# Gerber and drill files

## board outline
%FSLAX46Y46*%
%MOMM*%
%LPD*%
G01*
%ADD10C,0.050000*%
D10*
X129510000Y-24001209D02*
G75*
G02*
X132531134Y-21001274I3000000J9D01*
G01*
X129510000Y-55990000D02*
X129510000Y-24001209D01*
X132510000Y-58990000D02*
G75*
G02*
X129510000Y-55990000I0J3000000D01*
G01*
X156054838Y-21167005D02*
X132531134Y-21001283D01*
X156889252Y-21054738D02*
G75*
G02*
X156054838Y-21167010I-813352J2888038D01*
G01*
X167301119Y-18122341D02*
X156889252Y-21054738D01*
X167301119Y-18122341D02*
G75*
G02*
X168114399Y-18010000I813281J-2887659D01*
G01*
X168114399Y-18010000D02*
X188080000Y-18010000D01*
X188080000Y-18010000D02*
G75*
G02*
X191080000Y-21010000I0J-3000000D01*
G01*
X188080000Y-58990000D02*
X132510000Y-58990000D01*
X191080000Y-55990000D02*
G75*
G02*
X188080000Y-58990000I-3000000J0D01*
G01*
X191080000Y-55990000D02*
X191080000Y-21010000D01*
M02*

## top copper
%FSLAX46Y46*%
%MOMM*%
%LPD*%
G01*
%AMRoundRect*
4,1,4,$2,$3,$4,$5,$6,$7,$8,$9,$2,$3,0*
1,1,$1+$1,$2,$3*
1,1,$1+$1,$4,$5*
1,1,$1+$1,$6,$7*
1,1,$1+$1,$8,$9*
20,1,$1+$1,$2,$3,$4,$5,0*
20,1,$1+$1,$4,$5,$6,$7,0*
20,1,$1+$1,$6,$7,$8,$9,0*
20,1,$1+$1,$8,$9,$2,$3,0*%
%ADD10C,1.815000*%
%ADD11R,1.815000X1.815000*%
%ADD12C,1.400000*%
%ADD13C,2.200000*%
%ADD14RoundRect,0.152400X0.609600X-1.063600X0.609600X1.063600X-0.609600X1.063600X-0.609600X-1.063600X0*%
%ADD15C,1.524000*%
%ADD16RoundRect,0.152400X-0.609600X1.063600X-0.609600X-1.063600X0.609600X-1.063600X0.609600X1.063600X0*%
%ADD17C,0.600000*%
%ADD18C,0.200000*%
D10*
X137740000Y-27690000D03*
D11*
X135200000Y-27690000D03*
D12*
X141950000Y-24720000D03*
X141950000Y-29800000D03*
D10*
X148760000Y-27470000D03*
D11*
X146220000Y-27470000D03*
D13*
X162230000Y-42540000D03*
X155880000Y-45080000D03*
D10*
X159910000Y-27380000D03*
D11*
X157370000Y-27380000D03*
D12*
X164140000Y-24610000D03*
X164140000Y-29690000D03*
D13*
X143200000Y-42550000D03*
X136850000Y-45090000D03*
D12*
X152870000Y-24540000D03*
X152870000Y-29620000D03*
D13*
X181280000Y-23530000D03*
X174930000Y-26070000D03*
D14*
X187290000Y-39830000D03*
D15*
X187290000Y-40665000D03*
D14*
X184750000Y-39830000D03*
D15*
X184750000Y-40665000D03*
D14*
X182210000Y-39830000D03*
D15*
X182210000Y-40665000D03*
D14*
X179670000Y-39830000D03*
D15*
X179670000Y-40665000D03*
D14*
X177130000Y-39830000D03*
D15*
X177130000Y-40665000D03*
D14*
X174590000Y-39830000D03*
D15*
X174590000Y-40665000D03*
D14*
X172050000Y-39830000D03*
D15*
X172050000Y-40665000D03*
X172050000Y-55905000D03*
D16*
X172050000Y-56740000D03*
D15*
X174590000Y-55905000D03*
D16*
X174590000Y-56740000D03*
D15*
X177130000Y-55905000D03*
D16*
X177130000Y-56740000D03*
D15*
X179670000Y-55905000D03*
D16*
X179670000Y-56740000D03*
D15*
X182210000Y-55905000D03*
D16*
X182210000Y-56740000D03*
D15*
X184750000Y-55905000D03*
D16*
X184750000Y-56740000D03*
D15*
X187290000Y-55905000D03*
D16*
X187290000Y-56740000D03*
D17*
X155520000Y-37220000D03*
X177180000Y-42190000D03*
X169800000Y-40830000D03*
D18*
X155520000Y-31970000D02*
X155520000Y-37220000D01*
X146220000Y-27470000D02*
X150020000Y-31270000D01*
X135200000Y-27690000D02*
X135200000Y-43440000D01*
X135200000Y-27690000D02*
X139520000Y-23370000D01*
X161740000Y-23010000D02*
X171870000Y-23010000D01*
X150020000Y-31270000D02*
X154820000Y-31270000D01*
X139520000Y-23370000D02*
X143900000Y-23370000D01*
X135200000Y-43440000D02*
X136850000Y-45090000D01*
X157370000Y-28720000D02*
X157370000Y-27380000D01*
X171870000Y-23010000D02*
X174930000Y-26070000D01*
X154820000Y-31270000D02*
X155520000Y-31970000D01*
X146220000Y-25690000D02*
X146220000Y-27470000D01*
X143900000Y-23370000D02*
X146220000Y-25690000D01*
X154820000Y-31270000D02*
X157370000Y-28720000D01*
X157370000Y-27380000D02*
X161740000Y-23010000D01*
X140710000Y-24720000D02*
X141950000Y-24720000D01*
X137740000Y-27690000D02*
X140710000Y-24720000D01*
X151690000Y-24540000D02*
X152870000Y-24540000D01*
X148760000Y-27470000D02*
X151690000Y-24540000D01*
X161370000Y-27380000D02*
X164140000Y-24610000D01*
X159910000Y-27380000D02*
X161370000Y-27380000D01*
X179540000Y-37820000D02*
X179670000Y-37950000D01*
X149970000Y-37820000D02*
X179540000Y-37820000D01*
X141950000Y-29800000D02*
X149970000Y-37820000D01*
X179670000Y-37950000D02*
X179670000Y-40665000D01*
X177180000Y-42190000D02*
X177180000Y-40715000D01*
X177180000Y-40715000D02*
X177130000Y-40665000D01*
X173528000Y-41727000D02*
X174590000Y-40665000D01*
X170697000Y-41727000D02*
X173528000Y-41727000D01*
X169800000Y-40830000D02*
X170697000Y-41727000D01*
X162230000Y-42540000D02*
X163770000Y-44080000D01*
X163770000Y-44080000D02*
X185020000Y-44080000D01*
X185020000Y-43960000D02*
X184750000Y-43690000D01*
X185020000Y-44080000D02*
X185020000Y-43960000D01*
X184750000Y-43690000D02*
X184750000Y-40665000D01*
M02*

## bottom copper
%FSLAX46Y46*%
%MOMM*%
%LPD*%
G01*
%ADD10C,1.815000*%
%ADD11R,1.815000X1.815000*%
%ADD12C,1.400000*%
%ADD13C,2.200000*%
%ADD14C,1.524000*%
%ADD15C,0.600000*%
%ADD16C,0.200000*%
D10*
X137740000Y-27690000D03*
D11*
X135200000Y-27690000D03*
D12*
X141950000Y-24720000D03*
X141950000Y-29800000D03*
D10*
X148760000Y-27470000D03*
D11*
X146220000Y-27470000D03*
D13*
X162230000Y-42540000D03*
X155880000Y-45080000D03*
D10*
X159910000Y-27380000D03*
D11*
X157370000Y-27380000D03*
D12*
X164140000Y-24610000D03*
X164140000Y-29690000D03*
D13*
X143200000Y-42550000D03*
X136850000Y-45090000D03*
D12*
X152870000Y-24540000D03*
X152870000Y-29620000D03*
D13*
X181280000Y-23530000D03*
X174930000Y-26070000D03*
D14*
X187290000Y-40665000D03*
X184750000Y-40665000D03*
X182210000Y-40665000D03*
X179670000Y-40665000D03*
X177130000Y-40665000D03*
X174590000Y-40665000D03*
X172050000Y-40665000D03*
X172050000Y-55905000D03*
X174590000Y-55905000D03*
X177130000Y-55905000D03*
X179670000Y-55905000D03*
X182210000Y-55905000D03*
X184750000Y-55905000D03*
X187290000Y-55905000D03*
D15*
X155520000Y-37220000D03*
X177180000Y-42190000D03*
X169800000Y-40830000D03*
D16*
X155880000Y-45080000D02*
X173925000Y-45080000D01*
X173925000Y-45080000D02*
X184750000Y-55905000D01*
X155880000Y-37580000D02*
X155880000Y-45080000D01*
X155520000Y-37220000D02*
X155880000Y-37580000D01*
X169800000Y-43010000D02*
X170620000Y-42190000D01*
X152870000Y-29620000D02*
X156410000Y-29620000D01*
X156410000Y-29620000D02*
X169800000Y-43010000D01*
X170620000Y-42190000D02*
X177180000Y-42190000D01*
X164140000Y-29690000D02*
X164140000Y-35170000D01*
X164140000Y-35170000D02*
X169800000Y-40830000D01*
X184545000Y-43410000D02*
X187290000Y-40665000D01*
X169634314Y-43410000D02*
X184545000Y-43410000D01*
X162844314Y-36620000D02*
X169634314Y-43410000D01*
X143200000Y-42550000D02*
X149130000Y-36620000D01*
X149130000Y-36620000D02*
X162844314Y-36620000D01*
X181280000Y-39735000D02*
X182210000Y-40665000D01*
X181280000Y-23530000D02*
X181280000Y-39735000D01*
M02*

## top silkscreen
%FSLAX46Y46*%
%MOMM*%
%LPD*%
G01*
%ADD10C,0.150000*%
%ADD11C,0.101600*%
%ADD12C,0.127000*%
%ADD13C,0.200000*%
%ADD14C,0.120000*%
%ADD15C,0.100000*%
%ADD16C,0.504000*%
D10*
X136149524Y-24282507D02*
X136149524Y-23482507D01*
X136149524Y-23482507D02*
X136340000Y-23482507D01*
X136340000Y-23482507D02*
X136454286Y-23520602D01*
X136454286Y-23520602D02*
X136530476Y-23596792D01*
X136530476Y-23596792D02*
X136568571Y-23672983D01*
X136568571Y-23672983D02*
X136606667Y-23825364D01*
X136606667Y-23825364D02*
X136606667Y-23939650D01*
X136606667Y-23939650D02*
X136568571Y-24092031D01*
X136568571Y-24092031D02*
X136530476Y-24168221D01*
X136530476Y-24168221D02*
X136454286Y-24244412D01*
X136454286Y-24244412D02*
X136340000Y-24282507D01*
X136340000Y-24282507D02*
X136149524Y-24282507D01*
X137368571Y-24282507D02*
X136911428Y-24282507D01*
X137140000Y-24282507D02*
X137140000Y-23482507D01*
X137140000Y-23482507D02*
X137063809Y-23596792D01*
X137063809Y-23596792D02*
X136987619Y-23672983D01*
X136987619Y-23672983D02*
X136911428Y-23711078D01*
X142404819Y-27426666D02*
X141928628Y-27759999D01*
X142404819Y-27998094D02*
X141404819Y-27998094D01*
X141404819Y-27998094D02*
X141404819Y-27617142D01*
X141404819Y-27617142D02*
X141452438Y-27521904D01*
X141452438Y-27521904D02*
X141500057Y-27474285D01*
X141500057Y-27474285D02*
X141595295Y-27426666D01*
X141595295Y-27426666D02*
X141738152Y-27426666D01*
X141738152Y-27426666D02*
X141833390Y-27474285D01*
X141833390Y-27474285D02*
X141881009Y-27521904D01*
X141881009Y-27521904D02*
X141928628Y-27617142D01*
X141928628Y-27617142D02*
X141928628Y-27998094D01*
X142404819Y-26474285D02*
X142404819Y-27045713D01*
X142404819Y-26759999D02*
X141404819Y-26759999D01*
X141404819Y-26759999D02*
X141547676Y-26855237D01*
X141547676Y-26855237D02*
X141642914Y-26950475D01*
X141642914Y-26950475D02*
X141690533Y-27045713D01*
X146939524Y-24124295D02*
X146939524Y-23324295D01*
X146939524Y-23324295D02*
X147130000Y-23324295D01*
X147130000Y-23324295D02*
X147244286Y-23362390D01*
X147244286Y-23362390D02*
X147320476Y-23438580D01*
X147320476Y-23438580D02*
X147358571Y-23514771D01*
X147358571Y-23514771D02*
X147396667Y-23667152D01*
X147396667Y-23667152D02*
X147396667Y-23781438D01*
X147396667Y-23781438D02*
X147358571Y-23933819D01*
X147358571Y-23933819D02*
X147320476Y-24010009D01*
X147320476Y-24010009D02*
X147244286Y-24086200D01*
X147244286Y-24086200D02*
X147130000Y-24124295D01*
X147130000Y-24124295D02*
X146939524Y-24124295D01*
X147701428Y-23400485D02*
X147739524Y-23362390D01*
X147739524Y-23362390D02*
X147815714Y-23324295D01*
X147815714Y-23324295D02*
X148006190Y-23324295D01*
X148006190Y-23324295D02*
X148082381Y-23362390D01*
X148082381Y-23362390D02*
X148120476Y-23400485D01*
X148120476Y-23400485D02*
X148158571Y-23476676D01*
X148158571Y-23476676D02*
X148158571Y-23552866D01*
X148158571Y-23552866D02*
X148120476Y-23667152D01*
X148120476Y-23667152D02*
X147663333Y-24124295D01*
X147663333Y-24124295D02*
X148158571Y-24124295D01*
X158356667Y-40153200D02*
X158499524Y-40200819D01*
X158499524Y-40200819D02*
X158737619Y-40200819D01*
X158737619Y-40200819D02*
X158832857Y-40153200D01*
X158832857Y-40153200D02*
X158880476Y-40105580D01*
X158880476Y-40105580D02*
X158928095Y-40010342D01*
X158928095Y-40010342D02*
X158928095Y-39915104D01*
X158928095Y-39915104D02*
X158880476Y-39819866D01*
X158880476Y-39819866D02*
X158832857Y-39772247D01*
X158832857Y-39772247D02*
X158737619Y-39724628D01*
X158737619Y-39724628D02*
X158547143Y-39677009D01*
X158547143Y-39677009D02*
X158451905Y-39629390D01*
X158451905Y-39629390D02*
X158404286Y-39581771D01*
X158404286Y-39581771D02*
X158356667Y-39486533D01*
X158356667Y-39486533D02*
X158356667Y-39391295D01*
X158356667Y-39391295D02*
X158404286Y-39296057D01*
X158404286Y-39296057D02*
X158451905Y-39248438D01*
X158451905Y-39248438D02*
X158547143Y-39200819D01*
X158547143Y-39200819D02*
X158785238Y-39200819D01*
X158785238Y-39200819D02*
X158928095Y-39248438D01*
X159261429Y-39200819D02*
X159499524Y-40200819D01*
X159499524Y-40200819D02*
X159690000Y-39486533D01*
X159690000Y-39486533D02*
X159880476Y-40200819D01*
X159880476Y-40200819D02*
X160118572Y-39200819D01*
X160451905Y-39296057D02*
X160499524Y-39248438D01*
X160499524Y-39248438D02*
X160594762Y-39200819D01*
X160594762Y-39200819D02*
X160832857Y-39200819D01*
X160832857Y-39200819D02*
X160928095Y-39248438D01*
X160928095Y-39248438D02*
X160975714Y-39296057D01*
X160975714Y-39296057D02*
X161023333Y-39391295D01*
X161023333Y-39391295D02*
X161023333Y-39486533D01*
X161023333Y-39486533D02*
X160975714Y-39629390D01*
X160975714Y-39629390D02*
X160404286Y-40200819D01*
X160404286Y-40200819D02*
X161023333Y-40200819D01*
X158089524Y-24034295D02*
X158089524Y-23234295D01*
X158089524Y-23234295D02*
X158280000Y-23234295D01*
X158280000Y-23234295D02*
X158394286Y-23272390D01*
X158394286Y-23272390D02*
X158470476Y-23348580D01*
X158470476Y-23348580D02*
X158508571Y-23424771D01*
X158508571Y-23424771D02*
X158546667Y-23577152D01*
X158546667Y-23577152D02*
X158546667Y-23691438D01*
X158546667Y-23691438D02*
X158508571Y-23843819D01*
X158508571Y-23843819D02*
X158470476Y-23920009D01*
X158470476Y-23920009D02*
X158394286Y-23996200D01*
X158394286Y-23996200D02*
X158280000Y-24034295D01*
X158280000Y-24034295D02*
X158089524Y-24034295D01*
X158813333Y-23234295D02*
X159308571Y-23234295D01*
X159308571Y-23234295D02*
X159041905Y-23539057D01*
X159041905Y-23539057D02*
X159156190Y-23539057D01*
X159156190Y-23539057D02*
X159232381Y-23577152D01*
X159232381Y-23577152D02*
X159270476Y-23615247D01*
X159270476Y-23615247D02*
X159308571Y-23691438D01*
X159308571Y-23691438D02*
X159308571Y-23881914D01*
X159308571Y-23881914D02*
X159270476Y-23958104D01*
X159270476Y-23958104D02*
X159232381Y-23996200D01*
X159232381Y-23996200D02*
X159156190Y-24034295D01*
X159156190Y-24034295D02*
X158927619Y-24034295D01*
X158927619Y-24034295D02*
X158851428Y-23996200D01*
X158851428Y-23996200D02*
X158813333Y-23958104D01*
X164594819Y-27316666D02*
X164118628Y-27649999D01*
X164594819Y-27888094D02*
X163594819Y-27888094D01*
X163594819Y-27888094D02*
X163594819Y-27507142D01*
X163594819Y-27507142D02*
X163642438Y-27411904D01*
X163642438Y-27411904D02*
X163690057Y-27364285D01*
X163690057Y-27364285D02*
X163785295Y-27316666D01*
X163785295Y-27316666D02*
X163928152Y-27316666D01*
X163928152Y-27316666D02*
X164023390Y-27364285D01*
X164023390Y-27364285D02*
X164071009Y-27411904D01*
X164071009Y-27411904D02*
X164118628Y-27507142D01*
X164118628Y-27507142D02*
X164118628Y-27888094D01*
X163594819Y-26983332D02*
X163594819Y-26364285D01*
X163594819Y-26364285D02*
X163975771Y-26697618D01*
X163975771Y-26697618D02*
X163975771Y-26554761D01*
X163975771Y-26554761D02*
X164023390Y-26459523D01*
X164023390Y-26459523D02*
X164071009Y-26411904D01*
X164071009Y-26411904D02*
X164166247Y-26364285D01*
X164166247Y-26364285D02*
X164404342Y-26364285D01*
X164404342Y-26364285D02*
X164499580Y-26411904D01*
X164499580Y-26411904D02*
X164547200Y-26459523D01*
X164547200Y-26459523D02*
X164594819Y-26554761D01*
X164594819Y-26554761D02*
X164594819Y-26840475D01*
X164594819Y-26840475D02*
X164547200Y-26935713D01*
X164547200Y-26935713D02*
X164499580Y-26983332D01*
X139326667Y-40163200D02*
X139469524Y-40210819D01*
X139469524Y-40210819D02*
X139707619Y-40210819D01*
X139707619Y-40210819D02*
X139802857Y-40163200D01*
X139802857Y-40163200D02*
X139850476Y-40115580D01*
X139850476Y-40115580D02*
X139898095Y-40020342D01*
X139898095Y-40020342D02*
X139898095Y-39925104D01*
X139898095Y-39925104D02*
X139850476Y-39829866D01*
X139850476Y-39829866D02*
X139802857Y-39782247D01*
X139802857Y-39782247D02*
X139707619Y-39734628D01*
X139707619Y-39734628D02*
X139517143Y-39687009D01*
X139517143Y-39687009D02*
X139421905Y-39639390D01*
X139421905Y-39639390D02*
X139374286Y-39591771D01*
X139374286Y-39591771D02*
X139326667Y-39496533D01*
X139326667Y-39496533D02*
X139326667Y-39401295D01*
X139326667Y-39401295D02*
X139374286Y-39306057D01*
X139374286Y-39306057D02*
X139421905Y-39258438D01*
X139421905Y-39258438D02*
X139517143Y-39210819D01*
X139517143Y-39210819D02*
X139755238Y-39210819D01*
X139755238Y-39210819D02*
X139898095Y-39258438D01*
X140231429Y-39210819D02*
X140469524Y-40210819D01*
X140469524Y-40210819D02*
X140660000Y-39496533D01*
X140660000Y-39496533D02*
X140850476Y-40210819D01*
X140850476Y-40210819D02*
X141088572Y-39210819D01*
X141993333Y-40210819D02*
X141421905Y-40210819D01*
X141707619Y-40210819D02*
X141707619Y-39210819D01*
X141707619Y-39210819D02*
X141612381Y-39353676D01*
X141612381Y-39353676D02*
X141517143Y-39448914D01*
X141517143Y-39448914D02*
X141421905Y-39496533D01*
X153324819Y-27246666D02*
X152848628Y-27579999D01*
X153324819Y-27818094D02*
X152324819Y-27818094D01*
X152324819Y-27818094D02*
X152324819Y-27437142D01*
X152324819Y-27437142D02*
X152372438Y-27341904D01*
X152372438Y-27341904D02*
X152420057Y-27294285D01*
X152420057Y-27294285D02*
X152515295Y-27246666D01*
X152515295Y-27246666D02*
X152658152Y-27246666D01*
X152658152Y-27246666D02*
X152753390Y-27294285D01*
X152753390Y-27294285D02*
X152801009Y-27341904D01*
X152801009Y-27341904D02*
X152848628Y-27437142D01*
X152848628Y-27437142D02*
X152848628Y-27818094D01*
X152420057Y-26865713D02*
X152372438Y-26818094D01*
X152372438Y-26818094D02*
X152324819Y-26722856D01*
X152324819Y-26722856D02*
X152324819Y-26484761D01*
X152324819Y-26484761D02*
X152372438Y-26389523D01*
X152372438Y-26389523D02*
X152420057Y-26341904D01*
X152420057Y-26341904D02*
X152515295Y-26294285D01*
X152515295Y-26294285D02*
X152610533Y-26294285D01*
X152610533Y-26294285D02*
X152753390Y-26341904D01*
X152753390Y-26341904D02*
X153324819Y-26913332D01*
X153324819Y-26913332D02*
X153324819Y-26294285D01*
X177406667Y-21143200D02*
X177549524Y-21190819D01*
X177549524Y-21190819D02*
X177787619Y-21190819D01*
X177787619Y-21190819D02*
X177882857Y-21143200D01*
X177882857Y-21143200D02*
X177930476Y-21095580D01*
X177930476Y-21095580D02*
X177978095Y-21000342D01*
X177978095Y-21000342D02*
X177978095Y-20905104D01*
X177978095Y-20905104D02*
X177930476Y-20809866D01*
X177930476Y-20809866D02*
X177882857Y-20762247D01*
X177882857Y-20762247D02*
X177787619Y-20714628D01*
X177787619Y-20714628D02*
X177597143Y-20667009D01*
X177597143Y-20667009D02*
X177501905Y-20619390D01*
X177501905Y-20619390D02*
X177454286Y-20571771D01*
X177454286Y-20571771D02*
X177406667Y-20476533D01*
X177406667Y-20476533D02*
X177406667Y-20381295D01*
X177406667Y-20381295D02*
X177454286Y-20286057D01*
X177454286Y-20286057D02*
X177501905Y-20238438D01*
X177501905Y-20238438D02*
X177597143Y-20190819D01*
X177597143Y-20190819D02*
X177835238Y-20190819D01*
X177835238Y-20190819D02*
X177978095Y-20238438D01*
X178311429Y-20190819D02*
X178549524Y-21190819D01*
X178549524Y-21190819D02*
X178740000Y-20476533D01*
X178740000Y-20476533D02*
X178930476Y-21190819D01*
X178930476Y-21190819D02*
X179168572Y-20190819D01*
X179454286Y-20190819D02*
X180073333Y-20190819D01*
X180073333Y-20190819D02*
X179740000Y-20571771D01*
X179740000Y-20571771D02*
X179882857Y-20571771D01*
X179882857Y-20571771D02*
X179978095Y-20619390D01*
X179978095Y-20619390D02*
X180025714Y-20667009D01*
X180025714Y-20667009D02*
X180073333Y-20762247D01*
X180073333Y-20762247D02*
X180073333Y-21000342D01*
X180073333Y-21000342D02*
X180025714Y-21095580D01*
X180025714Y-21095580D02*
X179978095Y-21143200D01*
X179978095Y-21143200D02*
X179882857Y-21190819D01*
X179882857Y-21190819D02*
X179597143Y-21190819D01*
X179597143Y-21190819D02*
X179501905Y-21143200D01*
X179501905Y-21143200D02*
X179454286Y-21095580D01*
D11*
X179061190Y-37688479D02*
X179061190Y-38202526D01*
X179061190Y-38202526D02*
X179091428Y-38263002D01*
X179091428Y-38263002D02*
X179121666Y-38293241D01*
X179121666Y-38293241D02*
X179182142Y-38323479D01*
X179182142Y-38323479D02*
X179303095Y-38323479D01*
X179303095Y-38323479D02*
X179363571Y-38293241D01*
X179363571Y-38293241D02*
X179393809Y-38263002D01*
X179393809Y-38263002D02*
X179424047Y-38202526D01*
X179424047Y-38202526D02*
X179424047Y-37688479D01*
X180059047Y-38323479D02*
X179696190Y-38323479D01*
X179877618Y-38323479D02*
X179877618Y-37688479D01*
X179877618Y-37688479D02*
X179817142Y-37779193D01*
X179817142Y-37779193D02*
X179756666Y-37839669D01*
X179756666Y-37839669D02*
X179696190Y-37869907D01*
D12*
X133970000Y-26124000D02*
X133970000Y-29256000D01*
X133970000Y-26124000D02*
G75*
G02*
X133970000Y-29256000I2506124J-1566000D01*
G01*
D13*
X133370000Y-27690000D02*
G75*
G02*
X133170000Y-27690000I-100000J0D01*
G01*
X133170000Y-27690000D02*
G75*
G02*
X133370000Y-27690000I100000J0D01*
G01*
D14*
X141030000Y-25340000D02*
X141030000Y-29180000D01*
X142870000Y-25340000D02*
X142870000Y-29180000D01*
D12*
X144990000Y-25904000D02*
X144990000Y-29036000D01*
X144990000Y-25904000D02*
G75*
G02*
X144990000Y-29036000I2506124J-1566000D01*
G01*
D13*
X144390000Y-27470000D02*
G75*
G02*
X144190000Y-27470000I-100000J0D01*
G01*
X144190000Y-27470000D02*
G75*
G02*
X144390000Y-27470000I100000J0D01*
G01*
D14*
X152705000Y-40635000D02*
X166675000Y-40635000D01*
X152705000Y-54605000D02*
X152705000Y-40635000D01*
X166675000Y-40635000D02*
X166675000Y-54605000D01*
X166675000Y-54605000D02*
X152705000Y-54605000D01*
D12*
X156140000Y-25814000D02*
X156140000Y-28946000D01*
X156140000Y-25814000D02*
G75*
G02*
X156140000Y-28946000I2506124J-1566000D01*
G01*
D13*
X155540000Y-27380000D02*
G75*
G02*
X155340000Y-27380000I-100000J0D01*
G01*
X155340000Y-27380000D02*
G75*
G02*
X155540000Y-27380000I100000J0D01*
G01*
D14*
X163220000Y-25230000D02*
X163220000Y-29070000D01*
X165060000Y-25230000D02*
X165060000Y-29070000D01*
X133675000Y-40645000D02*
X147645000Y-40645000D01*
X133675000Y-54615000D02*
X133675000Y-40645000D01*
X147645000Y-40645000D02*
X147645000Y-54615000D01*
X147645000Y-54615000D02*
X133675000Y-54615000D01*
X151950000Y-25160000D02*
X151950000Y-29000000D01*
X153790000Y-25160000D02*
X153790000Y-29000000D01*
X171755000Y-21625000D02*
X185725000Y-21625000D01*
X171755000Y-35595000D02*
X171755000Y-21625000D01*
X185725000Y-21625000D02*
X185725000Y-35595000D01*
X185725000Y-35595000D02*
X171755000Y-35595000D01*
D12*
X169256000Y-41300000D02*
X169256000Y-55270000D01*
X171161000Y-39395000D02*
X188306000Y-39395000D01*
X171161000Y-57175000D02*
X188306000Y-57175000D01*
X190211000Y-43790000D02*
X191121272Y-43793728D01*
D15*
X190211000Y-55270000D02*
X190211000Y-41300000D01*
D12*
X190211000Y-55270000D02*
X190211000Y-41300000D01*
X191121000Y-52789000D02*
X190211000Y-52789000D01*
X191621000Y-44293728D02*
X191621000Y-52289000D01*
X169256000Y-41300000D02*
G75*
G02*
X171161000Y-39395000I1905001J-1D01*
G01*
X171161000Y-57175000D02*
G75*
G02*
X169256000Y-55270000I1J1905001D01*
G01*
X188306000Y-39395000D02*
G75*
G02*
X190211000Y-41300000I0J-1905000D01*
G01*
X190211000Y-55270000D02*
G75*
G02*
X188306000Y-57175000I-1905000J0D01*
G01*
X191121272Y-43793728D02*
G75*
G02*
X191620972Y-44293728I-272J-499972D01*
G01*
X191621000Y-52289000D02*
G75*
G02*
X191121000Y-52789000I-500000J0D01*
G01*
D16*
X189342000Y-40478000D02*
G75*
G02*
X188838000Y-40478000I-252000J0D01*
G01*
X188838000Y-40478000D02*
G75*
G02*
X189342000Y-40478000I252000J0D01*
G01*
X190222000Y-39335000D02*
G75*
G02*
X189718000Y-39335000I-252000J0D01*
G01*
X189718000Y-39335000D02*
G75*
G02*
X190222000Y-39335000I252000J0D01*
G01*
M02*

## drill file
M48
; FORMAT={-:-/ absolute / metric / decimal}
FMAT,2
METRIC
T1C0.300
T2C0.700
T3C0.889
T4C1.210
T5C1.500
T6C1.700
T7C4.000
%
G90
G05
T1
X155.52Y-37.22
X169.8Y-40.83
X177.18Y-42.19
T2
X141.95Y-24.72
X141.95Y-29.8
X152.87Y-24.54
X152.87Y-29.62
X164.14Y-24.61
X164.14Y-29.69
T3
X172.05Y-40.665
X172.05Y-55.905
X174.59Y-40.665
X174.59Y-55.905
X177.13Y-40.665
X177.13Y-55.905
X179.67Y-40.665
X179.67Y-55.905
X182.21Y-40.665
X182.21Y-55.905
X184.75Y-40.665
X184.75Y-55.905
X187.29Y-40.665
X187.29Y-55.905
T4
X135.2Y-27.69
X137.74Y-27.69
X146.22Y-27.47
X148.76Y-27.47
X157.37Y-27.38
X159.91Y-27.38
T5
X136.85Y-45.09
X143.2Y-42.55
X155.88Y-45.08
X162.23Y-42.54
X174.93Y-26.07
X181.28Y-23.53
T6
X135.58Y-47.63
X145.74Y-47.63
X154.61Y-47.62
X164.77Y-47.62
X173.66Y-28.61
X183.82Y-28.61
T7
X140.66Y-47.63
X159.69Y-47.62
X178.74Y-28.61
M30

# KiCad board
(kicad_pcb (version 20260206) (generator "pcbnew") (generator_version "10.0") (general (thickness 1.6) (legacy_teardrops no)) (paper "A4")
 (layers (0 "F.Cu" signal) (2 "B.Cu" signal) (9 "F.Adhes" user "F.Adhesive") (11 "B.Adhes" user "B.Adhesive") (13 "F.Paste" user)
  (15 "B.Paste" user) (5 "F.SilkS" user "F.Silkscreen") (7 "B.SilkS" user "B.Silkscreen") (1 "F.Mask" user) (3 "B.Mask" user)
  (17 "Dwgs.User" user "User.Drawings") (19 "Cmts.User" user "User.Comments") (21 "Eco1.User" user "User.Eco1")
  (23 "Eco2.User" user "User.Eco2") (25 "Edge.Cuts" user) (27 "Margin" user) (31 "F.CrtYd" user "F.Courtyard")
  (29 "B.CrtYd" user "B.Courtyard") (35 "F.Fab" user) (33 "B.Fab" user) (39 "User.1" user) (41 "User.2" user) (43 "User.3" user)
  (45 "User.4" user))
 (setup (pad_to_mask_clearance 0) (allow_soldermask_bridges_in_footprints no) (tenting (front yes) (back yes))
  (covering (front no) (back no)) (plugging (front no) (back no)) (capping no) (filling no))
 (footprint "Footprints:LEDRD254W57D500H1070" (layer "F.Cu") (at 136.47 27.69)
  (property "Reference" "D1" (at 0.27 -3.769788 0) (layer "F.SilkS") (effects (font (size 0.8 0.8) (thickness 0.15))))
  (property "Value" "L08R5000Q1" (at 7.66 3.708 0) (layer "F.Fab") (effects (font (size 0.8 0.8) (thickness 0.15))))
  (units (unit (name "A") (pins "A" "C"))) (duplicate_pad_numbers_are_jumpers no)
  (fp_line (start -2.5 -1.566) (end -2.5 1.566) (stroke (width 0.127) (type solid)) (layer "F.SilkS"))
  (fp_arc (start -2.5 -1.566) (mid 2.961291 0) (end -2.5 1.566) (stroke (width 0.127) (type solid)) (layer "F.SilkS"))
  (fp_circle (center -3.2 0) (end -3.1 0) (stroke (width 0.2) (type solid)) (fill no) (layer "F.SilkS"))
  (pad "A" thru_hole circle (at 1.27 0) (size 1.815 1.815) (drill 1.21) (layers "*.Cu" "*.Mask") (remove_unused_layers no)
   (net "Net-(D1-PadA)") (solder_mask_margin 0.102))
  (pad "C" thru_hole rect (at -1.27 0) (size 1.815 1.815) (drill 1.21) (layers "*.Cu" "*.Mask") (remove_unused_layers no) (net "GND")
   (solder_mask_margin 0.102)))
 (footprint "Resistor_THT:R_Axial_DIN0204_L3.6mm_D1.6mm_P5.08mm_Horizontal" (layer "F.Cu") (at 141.95 24.72 -90)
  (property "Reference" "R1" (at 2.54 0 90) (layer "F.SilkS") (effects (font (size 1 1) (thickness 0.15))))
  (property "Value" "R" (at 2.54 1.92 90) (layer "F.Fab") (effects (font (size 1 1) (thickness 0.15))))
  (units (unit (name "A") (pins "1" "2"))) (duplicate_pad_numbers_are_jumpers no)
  (fp_line (start 0.62 0.92) (end 4.46 0.92) (stroke (width 0.12) (type solid)) (layer "F.SilkS"))
  (fp_line (start 0.62 -0.92) (end 4.46 -0.92) (stroke (width 0.12) (type solid)) (layer "F.SilkS"))
  (pad "1" thru_hole circle (at 0 0 270) (size 1.4 1.4) (drill 0.7) (layers "*.Cu" "*.Mask") (remove_unused_layers no) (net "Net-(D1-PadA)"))
  (pad "2" thru_hole circle (at 5.08 0 270) (size 1.4 1.4) (drill 0.7) (layers "*.Cu" "*.Mask") (remove_unused_layers no) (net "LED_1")))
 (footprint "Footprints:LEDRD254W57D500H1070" (layer "F.Cu") (at 147.49 27.47)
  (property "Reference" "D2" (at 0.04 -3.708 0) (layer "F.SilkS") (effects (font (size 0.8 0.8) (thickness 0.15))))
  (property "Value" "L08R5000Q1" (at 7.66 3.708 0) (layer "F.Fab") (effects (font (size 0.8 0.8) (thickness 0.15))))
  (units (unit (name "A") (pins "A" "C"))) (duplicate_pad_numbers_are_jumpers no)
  (fp_line (start -2.5 -1.566) (end -2.5 1.566) (stroke (width 0.127) (type solid)) (layer "F.SilkS"))
  (fp_arc (start -2.5 -1.566) (mid 2.961291 0) (end -2.5 1.566) (stroke (width 0.127) (type solid)) (layer "F.SilkS"))
  (fp_circle (center -3.2 0) (end -3.1 0) (stroke (width 0.2) (type solid)) (fill no) (layer "F.SilkS"))
  (pad "A" thru_hole circle (at 1.27 0) (size 1.815 1.815) (drill 1.21) (layers "*.Cu" "*.Mask") (remove_unused_layers no)
   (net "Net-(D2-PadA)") (solder_mask_margin 0.102))
  (pad "C" thru_hole rect (at -1.27 0) (size 1.815 1.815) (drill 1.21) (layers "*.Cu" "*.Mask") (remove_unused_layers no) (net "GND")
   (solder_mask_margin 0.102)))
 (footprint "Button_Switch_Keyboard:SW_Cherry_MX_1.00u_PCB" (layer "F.Cu") (at 162.23 42.54)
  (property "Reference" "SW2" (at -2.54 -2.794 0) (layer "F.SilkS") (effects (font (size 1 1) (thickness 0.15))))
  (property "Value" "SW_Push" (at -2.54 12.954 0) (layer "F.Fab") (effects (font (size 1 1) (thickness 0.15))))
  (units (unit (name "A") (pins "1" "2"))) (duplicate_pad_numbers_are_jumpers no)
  (fp_line (start -9.525 -1.905) (end 4.445 -1.905) (stroke (width 0.12) (type solid)) (layer "F.SilkS"))
  (fp_line (start -9.525 12.065) (end -9.525 -1.905) (stroke (width 0.12) (type solid)) (layer "F.SilkS"))
  (fp_line (start 4.445 -1.905) (end 4.445 12.065) (stroke (width 0.12) (type solid)) (layer "F.SilkS"))
  (fp_line (start 4.445 12.065) (end -9.525 12.065) (stroke (width 0.12) (type solid)) (layer "F.SilkS"))
  (pad "" np_thru_hole circle (at -7.62 5.08) (size 1.7 1.7) (drill 1.7) (layers "*.Cu" "*.Mask"))
  (pad "" np_thru_hole circle (at -2.54 5.08) (size 4 4) (drill 4) (layers "*.Cu" "*.Mask"))
  (pad "" np_thru_hole circle (at 2.54 5.08) (size 1.7 1.7) (drill 1.7) (layers "*.Cu" "*.Mask"))
  (pad "1" thru_hole circle (at 0 0) (size 2.2 2.2) (drill 1.5) (layers "*.Cu" "*.Mask") (remove_unused_layers no) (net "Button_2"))
  (pad "2" thru_hole circle (at -6.35 2.54) (size 2.2 2.2) (drill 1.5) (layers "*.Cu" "*.Mask") (remove_unused_layers no) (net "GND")))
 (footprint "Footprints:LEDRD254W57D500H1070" (layer "F.Cu") (at 158.64 27.38)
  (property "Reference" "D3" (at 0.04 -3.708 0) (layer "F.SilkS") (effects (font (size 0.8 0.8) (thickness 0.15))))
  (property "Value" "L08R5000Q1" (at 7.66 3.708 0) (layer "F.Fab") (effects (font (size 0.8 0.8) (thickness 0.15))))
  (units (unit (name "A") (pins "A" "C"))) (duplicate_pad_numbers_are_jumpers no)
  (fp_line (start -2.5 -1.566) (end -2.5 1.566) (stroke (width 0.127) (type solid)) (layer "F.SilkS"))
  (fp_arc (start -2.5 -1.566) (mid 2.961291 0) (end -2.5 1.566) (stroke (width 0.127) (type solid)) (layer "F.SilkS"))
  (fp_circle (center -3.2 0) (end -3.1 0) (stroke (width 0.2) (type solid)) (fill no) (layer "F.SilkS"))
  (pad "A" thru_hole circle (at 1.27 0) (size 1.815 1.815) (drill 1.21) (layers "*.Cu" "*.Mask") (remove_unused_layers no)
   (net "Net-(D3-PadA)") (solder_mask_margin 0.102))
  (pad "C" thru_hole rect (at -1.27 0) (size 1.815 1.815) (drill 1.21) (layers "*.Cu" "*.Mask") (remove_unused_layers no) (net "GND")
   (solder_mask_margin 0.102)))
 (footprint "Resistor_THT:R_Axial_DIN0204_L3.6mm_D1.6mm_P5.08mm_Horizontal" (layer "F.Cu") (at 164.14 24.61 -90)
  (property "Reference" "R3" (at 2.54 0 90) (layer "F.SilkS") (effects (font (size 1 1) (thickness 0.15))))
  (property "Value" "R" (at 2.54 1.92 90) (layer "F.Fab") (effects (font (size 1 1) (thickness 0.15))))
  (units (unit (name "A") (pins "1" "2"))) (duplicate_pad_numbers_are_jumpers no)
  (fp_line (start 0.62 0.92) (end 4.46 0.92) (stroke (width 0.12) (type solid)) (layer "F.SilkS"))
  (fp_line (start 0.62 -0.92) (end 4.46 -0.92) (stroke (width 0.12) (type solid)) (layer "F.SilkS"))
  (pad "1" thru_hole circle (at 0 0 270) (size 1.4 1.4) (drill 0.7) (layers "*.Cu" "*.Mask") (remove_unused_layers no) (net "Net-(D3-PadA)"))
  (pad "2" thru_hole circle (at 5.08 0 270) (size 1.4 1.4) (drill 0.7) (layers "*.Cu" "*.Mask") (remove_unused_layers no) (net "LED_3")))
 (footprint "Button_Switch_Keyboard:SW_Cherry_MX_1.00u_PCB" (layer "F.Cu") (at 143.2 42.55)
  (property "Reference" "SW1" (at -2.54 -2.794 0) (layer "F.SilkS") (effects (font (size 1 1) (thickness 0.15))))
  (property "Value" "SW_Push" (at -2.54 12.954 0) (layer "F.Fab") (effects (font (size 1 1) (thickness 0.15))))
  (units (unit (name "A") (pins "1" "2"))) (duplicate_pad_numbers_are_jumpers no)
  (fp_line (start -9.525 -1.905) (end 4.445 -1.905) (stroke (width 0.12) (type solid)) (layer "F.SilkS"))
  (fp_line (start -9.525 12.065) (end -9.525 -1.905) (stroke (width 0.12) (type solid)) (layer "F.SilkS"))
  (fp_line (start 4.445 -1.905) (end 4.445 12.065) (stroke (width 0.12) (type solid)) (layer "F.SilkS"))
  (fp_line (start 4.445 12.065) (end -9.525 12.065) (stroke (width 0.12) (type solid)) (layer "F.SilkS"))
  (pad "" np_thru_hole circle (at -7.62 5.08) (size 1.7 1.7) (drill 1.7) (layers "*.Cu" "*.Mask"))
  (pad "" np_thru_hole circle (at -2.54 5.08) (size 4 4) (drill 4) (layers "*.Cu" "*.Mask"))
  (pad "" np_thru_hole circle (at 2.54 5.08) (size 1.7 1.7) (drill 1.7) (layers "*.Cu" "*.Mask"))
  (pad "1" thru_hole circle (at 0 0) (size 2.2 2.2) (drill 1.5) (layers "*.Cu" "*.Mask") (remove_unused_layers no) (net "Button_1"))
  (pad "2" thru_hole circle (at -6.35 2.54) (size 2.2 2.2) (drill 1.5) (layers "*.Cu" "*.Mask") (remove_unused_layers no) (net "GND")))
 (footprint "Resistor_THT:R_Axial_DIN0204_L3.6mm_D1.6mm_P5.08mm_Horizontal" (layer "F.Cu") (at 152.87 24.54 -90)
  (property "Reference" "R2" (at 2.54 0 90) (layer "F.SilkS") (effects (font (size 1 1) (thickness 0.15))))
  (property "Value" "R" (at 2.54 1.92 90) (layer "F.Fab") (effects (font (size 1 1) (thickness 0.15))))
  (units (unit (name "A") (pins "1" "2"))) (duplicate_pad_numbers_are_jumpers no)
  (fp_line (start 0.62 0.92) (end 4.46 0.92) (stroke (width 0.12) (type solid)) (layer "F.SilkS"))
  (fp_line (start 0.62 -0.92) (end 4.46 -0.92) (stroke (width 0.12) (type solid)) (layer "F.SilkS"))
  (pad "1" thru_hole circle (at 0 0 270) (size 1.4 1.4) (drill 0.7) (layers "*.Cu" "*.Mask") (remove_unused_layers no) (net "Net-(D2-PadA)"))
  (pad "2" thru_hole circle (at 5.08 0 270) (size 1.4 1.4) (drill 0.7) (layers "*.Cu" "*.Mask") (remove_unused_layers no) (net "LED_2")))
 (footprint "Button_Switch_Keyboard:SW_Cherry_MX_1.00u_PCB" (layer "F.Cu") (at 181.28 23.53)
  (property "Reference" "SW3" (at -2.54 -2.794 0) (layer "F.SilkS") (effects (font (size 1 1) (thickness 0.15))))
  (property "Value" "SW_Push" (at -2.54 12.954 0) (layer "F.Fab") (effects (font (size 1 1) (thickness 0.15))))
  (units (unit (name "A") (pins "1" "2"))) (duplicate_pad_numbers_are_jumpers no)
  (fp_line (start -9.525 -1.905) (end 4.445 -1.905) (stroke (width 0.12) (type solid)) (layer "F.SilkS"))
  (fp_line (start -9.525 12.065) (end -9.525 -1.905) (stroke (width 0.12) (type solid)) (layer "F.SilkS"))
  (fp_line (start 4.445 -1.905) (end 4.445 12.065) (stroke (width 0.12) (type solid)) (layer "F.SilkS"))
  (fp_line (start 4.445 12.065) (end -9.525 12.065) (stroke (width 0.12) (type solid)) (layer "F.SilkS"))
  (pad "" np_thru_hole circle (at -7.62 5.08) (size 1.7 1.7) (drill 1.7) (layers "*.Cu" "*.Mask"))
  (pad "" np_thru_hole circle (at -2.54 5.08) (size 4 4) (drill 4) (layers "*.Cu" "*.Mask"))
  (pad "" np_thru_hole circle (at 2.54 5.08) (size 1.7 1.7) (drill 1.7) (layers "*.Cu" "*.Mask"))
  (pad "1" thru_hole circle (at 0 0) (size 2.2 2.2) (drill 1.5) (layers "*.Cu" "*.Mask") (remove_unused_layers no) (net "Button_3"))
  (pad "2" thru_hole circle (at -6.35 2.54) (size 2.2 2.2) (drill 1.5) (layers "*.Cu" "*.Mask") (remove_unused_layers no) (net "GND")))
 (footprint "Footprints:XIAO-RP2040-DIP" (layer "F.Cu") (at 179.67 48.285)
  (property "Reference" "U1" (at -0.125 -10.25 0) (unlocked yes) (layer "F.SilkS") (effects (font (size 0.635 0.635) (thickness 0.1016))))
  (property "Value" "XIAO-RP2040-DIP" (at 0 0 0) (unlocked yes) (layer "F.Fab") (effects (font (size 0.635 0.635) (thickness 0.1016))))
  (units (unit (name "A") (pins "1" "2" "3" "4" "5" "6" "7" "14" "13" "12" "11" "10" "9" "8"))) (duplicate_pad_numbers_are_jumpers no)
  (fp_line (start -10.414 -6.985) (end -10.414 6.985) (stroke (width 0.127) (type solid)) (layer "F.SilkS"))
  (fp_line (start -8.509 -8.89) (end 8.636 -8.89) (stroke (width 0.127) (type solid)) (layer "F.SilkS"))
  (fp_line (start -8.509 8.89) (end 8.636 8.89) (stroke (width 0.127) (type solid)) (layer "F.SilkS"))
  (fp_line (start 10.541 -4.495) (end 11.451272 -4.491272) (stroke (width 0.127) (type solid)) (layer "F.SilkS"))
  (fp_line (start 10.541 6.985) (end 10.541 -6.985) (stroke (width 0.1) (type solid)) (layer "F.SilkS"))
  (fp_line (start 10.541 6.985) (end 10.541 -6.985) (stroke (width 0.127) (type solid)) (layer "F.SilkS"))
  (fp_line (start 11.451 4.504) (end 10.541 4.504) (stroke (width 0.127) (type solid)) (layer "F.SilkS"))
  (fp_line (start 11.951 -3.991272) (end 11.951 4.004) (stroke (width 0.127) (type solid)) (layer "F.SilkS"))
  (fp_arc (start -10.414 -6.985) (mid -9.856038 -8.332038) (end -8.509 -8.89) (stroke (width 0.127) (type solid)) (layer "F.SilkS"))
  (fp_arc (start -8.509 8.89) (mid -9.856038 8.332038) (end -10.414 6.985) (stroke (width 0.127) (type solid)) (layer "F.SilkS"))
  (fp_arc (start 8.636 -8.89) (mid 9.983038 -8.332038) (end 10.541 -6.985) (stroke (width 0.127) (type solid)) (layer "F.SilkS"))
  (fp_arc (start 10.541 6.985) (mid 9.983038 8.332038) (end 8.636 8.89) (stroke (width 0.127) (type solid)) (layer "F.SilkS"))
  (fp_arc (start 11.451272 -4.491272) (mid 11.804644 -4.344724) (end 11.951 -3.991272) (stroke (width 0.127) (type default))
   (layer "F.SilkS"))
  (fp_arc (start 11.951 4.004) (mid 11.804553 4.357553) (end 11.451 4.504) (stroke (width 0.127) (type default)) (layer "F.SilkS"))
  (fp_circle (center 9.42 -7.807) (end 9.674 -7.807) (stroke (width 0.5) (type solid)) (fill yes) (layer "F.SilkS"))
  (fp_circle (center 10.3 -8.95) (end 10.554 -8.95) (stroke (width 0.5) (type solid)) (fill yes) (layer "F.SilkS"))
  (pad "1" smd roundrect (at 7.62 -8.455 90) (size 2.432 1.524) (layers "F.Cu" "F.Mask") (roundrect_rratio 0.1) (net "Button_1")
   (thermal_bridge_angle 45))
  (pad "1" thru_hole circle (at 7.62 -7.62 90) (size 1.524 1.524) (drill 0.889) (layers "*.Cu" "*.Mask") (remove_unused_layers no)
   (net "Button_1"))
  (pad "2" smd roundrect (at 5.08 -8.455 90) (size 2.432 1.524) (layers "F.Cu" "F.Mask") (roundrect_rratio 0.1) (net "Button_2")
   (thermal_bridge_angle 45))
  (pad "2" thru_hole circle (at 5.08 -7.62 90) (size 1.524 1.524) (drill 0.889) (layers "*.Cu" "*.Mask") (remove_unused_layers no)
   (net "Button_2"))
  (pad "3" smd roundrect (at 2.54 -8.455 90) (size 2.432 1.524) (layers "F.Cu" "F.Mask") (roundrect_rratio 0.1) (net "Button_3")
   (thermal_bridge_angle 45))
  (pad "3" thru_hole circle (at 2.54 -7.62 90) (size 1.524 1.524) (drill 0.889) (layers "*.Cu" "*.Mask") (remove_unused_layers no)
   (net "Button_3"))
  (pad "4" smd roundrect (at 0 -8.455 90) (size 2.432 1.524) (layers "F.Cu" "F.Mask") (roundrect_rratio 0.1) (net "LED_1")
   (thermal_bridge_angle 45))
  (pad "4" thru_hole circle (at 0 -7.62 90) (size 1.524 1.524) (drill 0.889) (layers "*.Cu" "*.Mask") (remove_unused_layers no)
   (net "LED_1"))
  (pad "5" smd roundrect (at -2.54 -8.455 90) (size 2.432 1.524) (layers "F.Cu" "F.Mask") (roundrect_rratio 0.1) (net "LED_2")
   (thermal_bridge_angle 45))
  (pad "5" thru_hole circle (at -2.54 -7.62 90) (size 1.524 1.524) (drill 0.889) (layers "*.Cu" "*.Mask") (remove_unused_layers no)
   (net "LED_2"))
  (pad "6" smd roundrect (at -5.08 -8.455 90) (size 2.432 1.524) (layers "F.Cu" "F.Mask") (roundrect_rratio 0.1) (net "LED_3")
   (thermal_bridge_angle 45))
  (pad "6" thru_hole circle (at -5.08 -7.62 90) (size 1.524 1.524) (drill 0.889) (layers "*.Cu" "*.Mask") (remove_unused_layers no)
   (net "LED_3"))
  (pad "7" smd roundrect (at -7.62 -8.455 90) (size 2.432 1.524) (layers "F.Cu" "F.Mask") (roundrect_rratio 0.1)
   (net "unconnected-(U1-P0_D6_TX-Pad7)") (thermal_bridge_angle 45))
  (pad "7" thru_hole circle (at -7.62 -7.62 90) (size 1.524 1.524) (drill 0.889) (layers "*.Cu" "*.Mask") (remove_unused_layers no)
   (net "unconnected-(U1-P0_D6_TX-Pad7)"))
  (pad "8" thru_hole circle (at -7.62 7.62 270) (size 1.524 1.524) (drill 0.889) (layers "*.Cu" "*.Mask") (remove_unused_layers no)
   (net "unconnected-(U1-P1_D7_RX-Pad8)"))
  (pad "8" smd roundrect (at -7.62 8.455 270) (size 2.432 1.524) (layers "F.Cu" "F.Mask") (roundrect_rratio 0.1)
   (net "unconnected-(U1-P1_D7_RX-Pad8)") (thermal_bridge_angle 45))
  (pad "9" thru_hole circle (at -5.08 7.62 270) (size 1.524 1.524) (drill 0.889) (layers "*.Cu" "*.Mask") (remove_unused_layers no)
   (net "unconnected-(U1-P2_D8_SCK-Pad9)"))
  (pad "9" smd roundrect (at -5.08 8.455 270) (size 2.432 1.524) (layers "F.Cu" "F.Mask") (roundrect_rratio 0.1)
   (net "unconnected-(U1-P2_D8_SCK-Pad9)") (thermal_bridge_angle 45))
  (pad "10" thru_hole circle (at -2.54 7.62 270) (size 1.524 1.524) (drill 0.889) (layers "*.Cu" "*.Mask") (remove_unused_layers no)
   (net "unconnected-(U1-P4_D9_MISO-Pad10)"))
  (pad "10" smd roundrect (at -2.54 8.455 270) (size 2.432 1.524) (layers "F.Cu" "F.Mask") (roundrect_rratio 0.1)
   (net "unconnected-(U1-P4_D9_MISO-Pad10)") (thermal_bridge_angle 45))
  (pad "11" thru_hole circle (at 0 7.62 270) (size 1.524 1.524) (drill 0.889) (layers "*.Cu" "*.Mask") (remove_unused_layers no)
   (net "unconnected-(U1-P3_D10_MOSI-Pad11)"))
  (pad "11" smd roundrect (at 0 8.455 270) (size 2.432 1.524) (layers "F.Cu" "F.Mask") (roundrect_rratio 0.1)
   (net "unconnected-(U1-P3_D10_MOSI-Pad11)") (thermal_bridge_angle 45))
  (pad "12" thru_hole circle (at 2.54 7.62 270) (size 1.524 1.524) (drill 0.889) (layers "*.Cu" "*.Mask") (remove_unused_layers no)
   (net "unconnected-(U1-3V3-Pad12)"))
  (pad "12" smd roundrect (at 2.54 8.455 270) (size 2.432 1.524) (layers "F.Cu" "F.Mask") (roundrect_rratio 0.1)
   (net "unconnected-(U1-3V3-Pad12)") (thermal_bridge_angle 45))
  (pad "13" thru_hole circle (at 5.08 7.62 270) (size 1.524 1.524) (drill 0.889) (layers "*.Cu" "*.Mask") (remove_unused_layers no)
   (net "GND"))
  (pad "13" smd roundrect (at 5.08 8.455 270) (size 2.432 1.524) (layers "F.Cu" "F.Mask") (roundrect_rratio 0.1) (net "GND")
   (thermal_bridge_angle 45))
  (pad "14" thru_hole circle (at 7.62 7.62 270) (size 1.524 1.524) (drill 0.889) (layers "*.Cu" "*.Mask") (remove_unused_layers no)
   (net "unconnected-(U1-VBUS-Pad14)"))
  (pad "14" smd roundrect (at 7.62 8.455 270) (size 2.432 1.524) (layers "F.Cu" "F.Mask") (roundrect_rratio 0.1)
   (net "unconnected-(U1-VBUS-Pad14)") (thermal_bridge_angle 45)))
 (gr_arc (start 129.51 24.001209) (mid 130.396162 21.872424) (end 132.531134 21.001283) (stroke (width 0.05) (type default))
  (layer "Edge.Cuts"))
 (gr_line (start 129.51 55.99) (end 129.51 24.001209) (stroke (width 0.05) (type default)) (layer "Edge.Cuts"))
 (gr_arc (start 132.51 58.99) (mid 130.38868 58.11132) (end 129.51 55.99) (stroke (width 0.05) (type default)) (layer "Edge.Cuts"))
 (gr_line (start 156.054838 21.167005) (end 132.531134 21.001283) (stroke (width 0.05) (type default)) (layer "Edge.Cuts"))
 (gr_arc (start 156.889252 21.054738) (mid 156.476003 21.140285) (end 156.054838 21.167005) (stroke (width 0.05) (type default))
  (layer "Edge.Cuts"))
 (gr_line (start 167.301119 18.122341) (end 156.889252 21.054738) (stroke (width 0.05) (type default)) (layer "Edge.Cuts"))
 (gr_arc (start 167.301119 18.122341) (mid 167.703898 18.038218) (end 168.114399 18.01) (stroke (width 0.05) (type default))
  (layer "Edge.Cuts"))
 (gr_line (start 168.114399 18.01) (end 188.08 18.01) (stroke (width 0.05) (type default)) (layer "Edge.Cuts"))
 (gr_arc (start 188.08 18.01) (mid 190.20132 18.88868) (end 191.08 21.01) (stroke (width 0.05) (type default)) (layer "Edge.Cuts"))
 (gr_line (start 188.08 58.99) (end 132.51 58.99) (stroke (width 0.05) (type default)) (layer "Edge.Cuts"))
 (gr_arc (start 191.08 55.99) (mid 190.20132 58.11132) (end 188.08 58.99) (stroke (width 0.05) (type default)) (layer "Edge.Cuts"))
 (gr_line (start 191.08 55.99) (end 191.08 21.01) (stroke (width 0.05) (type default)) (layer "Edge.Cuts"))
 (segment (start 155.52 31.97) (end 155.52 37.22) (width 0.2) (layer "F.Cu") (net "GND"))
 (segment (start 146.22 27.47) (end 150.02 31.27) (width 0.2) (layer "F.Cu") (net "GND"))
 (segment (start 135.2 27.69) (end 135.2 43.44) (width 0.2) (layer "F.Cu") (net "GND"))
 (segment (start 135.2 27.69) (end 139.52 23.37) (width 0.2) (layer "F.Cu") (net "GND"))
 (segment (start 161.74 23.01) (end 171.87 23.01) (width 0.2) (layer "F.Cu") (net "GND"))
 (segment (start 150.02 31.27) (end 154.82 31.27) (width 0.2) (layer "F.Cu") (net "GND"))
 (segment (start 139.52 23.37) (end 143.9 23.37) (width 0.2) (layer "F.Cu") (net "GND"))
 (segment (start 135.2 43.44) (end 136.85 45.09) (width 0.2) (layer "F.Cu") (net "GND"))
 (segment (start 157.37 28.72) (end 157.37 27.38) (width 0.2) (layer "F.Cu") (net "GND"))
 (segment (start 171.87 23.01) (end 174.93 26.07) (width 0.2) (layer "F.Cu") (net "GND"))
 (segment (start 154.82 31.27) (end 155.52 31.97) (width 0.2) (layer "F.Cu") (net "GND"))
 (segment (start 146.22 25.69) (end 146.22 27.47) (width 0.2) (layer "F.Cu") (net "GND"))
 (segment (start 143.9 23.37) (end 146.22 25.69) (width 0.2) (layer "F.Cu") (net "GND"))
 (segment (start 154.82 31.27) (end 157.37 28.72) (width 0.2) (layer "F.Cu") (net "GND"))
 (segment (start 157.37 27.38) (end 161.74 23.01) (width 0.2) (layer "F.Cu") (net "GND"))
 (via (at 155.52 37.22) (size 0.6) (drill 0.3) (layers "F.Cu" "B.Cu") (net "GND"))
 (segment (start 155.88 45.08) (end 173.925 45.08) (width 0.2) (layer "B.Cu") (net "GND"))
 (segment (start 173.925 45.08) (end 184.75 55.905) (width 0.2) (layer "B.Cu") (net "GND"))
 (segment (start 155.88 37.58) (end 155.88 45.08) (width 0.2) (layer "B.Cu") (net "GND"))
 (segment (start 155.52 37.22) (end 155.88 37.58) (width 0.2) (layer "B.Cu") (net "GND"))
 (segment (start 140.71 24.72) (end 141.95 24.72) (width 0.2) (layer "F.Cu") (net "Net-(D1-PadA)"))
 (segment (start 137.74 27.69) (end 140.71 24.72) (width 0.2) (layer "F.Cu") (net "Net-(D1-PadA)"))
 (segment (start 151.69 24.54) (end 152.87 24.54) (width 0.2) (layer "F.Cu") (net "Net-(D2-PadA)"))
 (segment (start 148.76 27.47) (end 151.69 24.54) (width 0.2) (layer "F.Cu") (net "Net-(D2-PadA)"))
 (segment (start 161.37 27.38) (end 164.14 24.61) (width 0.2) (layer "F.Cu") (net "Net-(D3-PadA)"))
 (segment (start 159.91 27.38) (end 161.37 27.38) (width 0.2) (layer "F.Cu") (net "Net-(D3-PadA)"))
 (segment (start 179.54 37.82) (end 179.67 37.95) (width 0.2) (layer "F.Cu") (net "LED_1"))
 (segment (start 149.97 37.82) (end 179.54 37.82) (width 0.2) (layer "F.Cu") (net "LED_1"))
 (segment (start 141.95 29.8) (end 149.97 37.82) (width 0.2) (layer "F.Cu") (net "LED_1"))
 (segment (start 179.67 37.95) (end 179.67 40.665) (width 0.2) (layer "F.Cu") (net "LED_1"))
 (segment (start 177.18 42.19) (end 177.18 40.715) (width 0.2) (layer "F.Cu") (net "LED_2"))
 (segment (start 177.18 40.715) (end 177.13 40.665) (width 0.2) (layer "F.Cu") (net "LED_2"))
 (via (at 177.18 42.19) (size 0.6) (drill 0.3) (layers "F.Cu" "B.Cu") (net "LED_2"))
 (segment (start 169.8 43.01) (end 170.62 42.19) (width 0.2) (layer "B.Cu") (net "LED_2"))
 (segment (start 152.87 29.62) (end 156.41 29.62) (width 0.2) (layer "B.Cu") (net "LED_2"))
 (segment (start 156.41 29.62) (end 169.8 43.01) (width 0.2) (layer "B.Cu") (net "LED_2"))
 (segment (start 170.62 42.19) (end 177.18 42.19) (width 0.2) (layer "B.Cu") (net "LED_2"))
 (segment (start 173.528 41.727) (end 174.59 40.665) (width 0.2) (layer "F.Cu") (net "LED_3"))
 (segment (start 170.697 41.727) (end 173.528 41.727) (width 0.2) (layer "F.Cu") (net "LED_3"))
 (segment (start 169.8 40.83) (end 170.697 41.727) (width 0.2) (layer "F.Cu") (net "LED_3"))
 (via (at 169.8 40.83) (size 0.6) (drill 0.3) (layers "F.Cu" "B.Cu") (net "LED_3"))
 (segment (start 164.14 29.69) (end 164.14 35.17) (width 0.2) (layer "B.Cu") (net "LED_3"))
 (segment (start 164.14 35.17) (end 169.8 40.83) (width 0.2) (layer "B.Cu") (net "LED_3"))
 (segment (start 184.545 43.41) (end 187.29 40.665) (width 0.2) (layer "B.Cu") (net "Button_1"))
 (segment (start 169.634314 43.41) (end 184.545 43.41) (width 0.2) (layer "B.Cu") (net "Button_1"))
 (segment (start 162.844314 36.62) (end 169.634314 43.41) (width 0.2) (layer "B.Cu") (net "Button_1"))
 (segment (start 143.2 42.55) (end 149.13 36.62) (width 0.2) (layer "B.Cu") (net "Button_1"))
 (segment (start 149.13 36.62) (end 162.844314 36.62) (width 0.2) (layer "B.Cu") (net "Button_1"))
 (segment (start 162.23 42.54) (end 163.77 44.08) (width 0.2) (layer "F.Cu") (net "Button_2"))
 (segment (start 163.77 44.08) (end 185.02 44.08) (width 0.2) (layer "F.Cu") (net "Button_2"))
 (segment (start 185.02 43.96) (end 184.75 43.69) (width 0.2) (layer "F.Cu") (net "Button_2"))
 (segment (start 185.02 44.08) (end 185.02 43.96) (width 0.2) (layer "F.Cu") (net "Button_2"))
 (segment (start 184.75 43.69) (end 184.75 40.665) (width 0.2) (layer "F.Cu") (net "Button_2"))
 (segment (start 181.28 39.735) (end 182.21 40.665) (width 0.2) (layer "B.Cu") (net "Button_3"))
 (segment (start 181.28 23.53) (end 181.28 39.735) (width 0.2) (layer "B.Cu") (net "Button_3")))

